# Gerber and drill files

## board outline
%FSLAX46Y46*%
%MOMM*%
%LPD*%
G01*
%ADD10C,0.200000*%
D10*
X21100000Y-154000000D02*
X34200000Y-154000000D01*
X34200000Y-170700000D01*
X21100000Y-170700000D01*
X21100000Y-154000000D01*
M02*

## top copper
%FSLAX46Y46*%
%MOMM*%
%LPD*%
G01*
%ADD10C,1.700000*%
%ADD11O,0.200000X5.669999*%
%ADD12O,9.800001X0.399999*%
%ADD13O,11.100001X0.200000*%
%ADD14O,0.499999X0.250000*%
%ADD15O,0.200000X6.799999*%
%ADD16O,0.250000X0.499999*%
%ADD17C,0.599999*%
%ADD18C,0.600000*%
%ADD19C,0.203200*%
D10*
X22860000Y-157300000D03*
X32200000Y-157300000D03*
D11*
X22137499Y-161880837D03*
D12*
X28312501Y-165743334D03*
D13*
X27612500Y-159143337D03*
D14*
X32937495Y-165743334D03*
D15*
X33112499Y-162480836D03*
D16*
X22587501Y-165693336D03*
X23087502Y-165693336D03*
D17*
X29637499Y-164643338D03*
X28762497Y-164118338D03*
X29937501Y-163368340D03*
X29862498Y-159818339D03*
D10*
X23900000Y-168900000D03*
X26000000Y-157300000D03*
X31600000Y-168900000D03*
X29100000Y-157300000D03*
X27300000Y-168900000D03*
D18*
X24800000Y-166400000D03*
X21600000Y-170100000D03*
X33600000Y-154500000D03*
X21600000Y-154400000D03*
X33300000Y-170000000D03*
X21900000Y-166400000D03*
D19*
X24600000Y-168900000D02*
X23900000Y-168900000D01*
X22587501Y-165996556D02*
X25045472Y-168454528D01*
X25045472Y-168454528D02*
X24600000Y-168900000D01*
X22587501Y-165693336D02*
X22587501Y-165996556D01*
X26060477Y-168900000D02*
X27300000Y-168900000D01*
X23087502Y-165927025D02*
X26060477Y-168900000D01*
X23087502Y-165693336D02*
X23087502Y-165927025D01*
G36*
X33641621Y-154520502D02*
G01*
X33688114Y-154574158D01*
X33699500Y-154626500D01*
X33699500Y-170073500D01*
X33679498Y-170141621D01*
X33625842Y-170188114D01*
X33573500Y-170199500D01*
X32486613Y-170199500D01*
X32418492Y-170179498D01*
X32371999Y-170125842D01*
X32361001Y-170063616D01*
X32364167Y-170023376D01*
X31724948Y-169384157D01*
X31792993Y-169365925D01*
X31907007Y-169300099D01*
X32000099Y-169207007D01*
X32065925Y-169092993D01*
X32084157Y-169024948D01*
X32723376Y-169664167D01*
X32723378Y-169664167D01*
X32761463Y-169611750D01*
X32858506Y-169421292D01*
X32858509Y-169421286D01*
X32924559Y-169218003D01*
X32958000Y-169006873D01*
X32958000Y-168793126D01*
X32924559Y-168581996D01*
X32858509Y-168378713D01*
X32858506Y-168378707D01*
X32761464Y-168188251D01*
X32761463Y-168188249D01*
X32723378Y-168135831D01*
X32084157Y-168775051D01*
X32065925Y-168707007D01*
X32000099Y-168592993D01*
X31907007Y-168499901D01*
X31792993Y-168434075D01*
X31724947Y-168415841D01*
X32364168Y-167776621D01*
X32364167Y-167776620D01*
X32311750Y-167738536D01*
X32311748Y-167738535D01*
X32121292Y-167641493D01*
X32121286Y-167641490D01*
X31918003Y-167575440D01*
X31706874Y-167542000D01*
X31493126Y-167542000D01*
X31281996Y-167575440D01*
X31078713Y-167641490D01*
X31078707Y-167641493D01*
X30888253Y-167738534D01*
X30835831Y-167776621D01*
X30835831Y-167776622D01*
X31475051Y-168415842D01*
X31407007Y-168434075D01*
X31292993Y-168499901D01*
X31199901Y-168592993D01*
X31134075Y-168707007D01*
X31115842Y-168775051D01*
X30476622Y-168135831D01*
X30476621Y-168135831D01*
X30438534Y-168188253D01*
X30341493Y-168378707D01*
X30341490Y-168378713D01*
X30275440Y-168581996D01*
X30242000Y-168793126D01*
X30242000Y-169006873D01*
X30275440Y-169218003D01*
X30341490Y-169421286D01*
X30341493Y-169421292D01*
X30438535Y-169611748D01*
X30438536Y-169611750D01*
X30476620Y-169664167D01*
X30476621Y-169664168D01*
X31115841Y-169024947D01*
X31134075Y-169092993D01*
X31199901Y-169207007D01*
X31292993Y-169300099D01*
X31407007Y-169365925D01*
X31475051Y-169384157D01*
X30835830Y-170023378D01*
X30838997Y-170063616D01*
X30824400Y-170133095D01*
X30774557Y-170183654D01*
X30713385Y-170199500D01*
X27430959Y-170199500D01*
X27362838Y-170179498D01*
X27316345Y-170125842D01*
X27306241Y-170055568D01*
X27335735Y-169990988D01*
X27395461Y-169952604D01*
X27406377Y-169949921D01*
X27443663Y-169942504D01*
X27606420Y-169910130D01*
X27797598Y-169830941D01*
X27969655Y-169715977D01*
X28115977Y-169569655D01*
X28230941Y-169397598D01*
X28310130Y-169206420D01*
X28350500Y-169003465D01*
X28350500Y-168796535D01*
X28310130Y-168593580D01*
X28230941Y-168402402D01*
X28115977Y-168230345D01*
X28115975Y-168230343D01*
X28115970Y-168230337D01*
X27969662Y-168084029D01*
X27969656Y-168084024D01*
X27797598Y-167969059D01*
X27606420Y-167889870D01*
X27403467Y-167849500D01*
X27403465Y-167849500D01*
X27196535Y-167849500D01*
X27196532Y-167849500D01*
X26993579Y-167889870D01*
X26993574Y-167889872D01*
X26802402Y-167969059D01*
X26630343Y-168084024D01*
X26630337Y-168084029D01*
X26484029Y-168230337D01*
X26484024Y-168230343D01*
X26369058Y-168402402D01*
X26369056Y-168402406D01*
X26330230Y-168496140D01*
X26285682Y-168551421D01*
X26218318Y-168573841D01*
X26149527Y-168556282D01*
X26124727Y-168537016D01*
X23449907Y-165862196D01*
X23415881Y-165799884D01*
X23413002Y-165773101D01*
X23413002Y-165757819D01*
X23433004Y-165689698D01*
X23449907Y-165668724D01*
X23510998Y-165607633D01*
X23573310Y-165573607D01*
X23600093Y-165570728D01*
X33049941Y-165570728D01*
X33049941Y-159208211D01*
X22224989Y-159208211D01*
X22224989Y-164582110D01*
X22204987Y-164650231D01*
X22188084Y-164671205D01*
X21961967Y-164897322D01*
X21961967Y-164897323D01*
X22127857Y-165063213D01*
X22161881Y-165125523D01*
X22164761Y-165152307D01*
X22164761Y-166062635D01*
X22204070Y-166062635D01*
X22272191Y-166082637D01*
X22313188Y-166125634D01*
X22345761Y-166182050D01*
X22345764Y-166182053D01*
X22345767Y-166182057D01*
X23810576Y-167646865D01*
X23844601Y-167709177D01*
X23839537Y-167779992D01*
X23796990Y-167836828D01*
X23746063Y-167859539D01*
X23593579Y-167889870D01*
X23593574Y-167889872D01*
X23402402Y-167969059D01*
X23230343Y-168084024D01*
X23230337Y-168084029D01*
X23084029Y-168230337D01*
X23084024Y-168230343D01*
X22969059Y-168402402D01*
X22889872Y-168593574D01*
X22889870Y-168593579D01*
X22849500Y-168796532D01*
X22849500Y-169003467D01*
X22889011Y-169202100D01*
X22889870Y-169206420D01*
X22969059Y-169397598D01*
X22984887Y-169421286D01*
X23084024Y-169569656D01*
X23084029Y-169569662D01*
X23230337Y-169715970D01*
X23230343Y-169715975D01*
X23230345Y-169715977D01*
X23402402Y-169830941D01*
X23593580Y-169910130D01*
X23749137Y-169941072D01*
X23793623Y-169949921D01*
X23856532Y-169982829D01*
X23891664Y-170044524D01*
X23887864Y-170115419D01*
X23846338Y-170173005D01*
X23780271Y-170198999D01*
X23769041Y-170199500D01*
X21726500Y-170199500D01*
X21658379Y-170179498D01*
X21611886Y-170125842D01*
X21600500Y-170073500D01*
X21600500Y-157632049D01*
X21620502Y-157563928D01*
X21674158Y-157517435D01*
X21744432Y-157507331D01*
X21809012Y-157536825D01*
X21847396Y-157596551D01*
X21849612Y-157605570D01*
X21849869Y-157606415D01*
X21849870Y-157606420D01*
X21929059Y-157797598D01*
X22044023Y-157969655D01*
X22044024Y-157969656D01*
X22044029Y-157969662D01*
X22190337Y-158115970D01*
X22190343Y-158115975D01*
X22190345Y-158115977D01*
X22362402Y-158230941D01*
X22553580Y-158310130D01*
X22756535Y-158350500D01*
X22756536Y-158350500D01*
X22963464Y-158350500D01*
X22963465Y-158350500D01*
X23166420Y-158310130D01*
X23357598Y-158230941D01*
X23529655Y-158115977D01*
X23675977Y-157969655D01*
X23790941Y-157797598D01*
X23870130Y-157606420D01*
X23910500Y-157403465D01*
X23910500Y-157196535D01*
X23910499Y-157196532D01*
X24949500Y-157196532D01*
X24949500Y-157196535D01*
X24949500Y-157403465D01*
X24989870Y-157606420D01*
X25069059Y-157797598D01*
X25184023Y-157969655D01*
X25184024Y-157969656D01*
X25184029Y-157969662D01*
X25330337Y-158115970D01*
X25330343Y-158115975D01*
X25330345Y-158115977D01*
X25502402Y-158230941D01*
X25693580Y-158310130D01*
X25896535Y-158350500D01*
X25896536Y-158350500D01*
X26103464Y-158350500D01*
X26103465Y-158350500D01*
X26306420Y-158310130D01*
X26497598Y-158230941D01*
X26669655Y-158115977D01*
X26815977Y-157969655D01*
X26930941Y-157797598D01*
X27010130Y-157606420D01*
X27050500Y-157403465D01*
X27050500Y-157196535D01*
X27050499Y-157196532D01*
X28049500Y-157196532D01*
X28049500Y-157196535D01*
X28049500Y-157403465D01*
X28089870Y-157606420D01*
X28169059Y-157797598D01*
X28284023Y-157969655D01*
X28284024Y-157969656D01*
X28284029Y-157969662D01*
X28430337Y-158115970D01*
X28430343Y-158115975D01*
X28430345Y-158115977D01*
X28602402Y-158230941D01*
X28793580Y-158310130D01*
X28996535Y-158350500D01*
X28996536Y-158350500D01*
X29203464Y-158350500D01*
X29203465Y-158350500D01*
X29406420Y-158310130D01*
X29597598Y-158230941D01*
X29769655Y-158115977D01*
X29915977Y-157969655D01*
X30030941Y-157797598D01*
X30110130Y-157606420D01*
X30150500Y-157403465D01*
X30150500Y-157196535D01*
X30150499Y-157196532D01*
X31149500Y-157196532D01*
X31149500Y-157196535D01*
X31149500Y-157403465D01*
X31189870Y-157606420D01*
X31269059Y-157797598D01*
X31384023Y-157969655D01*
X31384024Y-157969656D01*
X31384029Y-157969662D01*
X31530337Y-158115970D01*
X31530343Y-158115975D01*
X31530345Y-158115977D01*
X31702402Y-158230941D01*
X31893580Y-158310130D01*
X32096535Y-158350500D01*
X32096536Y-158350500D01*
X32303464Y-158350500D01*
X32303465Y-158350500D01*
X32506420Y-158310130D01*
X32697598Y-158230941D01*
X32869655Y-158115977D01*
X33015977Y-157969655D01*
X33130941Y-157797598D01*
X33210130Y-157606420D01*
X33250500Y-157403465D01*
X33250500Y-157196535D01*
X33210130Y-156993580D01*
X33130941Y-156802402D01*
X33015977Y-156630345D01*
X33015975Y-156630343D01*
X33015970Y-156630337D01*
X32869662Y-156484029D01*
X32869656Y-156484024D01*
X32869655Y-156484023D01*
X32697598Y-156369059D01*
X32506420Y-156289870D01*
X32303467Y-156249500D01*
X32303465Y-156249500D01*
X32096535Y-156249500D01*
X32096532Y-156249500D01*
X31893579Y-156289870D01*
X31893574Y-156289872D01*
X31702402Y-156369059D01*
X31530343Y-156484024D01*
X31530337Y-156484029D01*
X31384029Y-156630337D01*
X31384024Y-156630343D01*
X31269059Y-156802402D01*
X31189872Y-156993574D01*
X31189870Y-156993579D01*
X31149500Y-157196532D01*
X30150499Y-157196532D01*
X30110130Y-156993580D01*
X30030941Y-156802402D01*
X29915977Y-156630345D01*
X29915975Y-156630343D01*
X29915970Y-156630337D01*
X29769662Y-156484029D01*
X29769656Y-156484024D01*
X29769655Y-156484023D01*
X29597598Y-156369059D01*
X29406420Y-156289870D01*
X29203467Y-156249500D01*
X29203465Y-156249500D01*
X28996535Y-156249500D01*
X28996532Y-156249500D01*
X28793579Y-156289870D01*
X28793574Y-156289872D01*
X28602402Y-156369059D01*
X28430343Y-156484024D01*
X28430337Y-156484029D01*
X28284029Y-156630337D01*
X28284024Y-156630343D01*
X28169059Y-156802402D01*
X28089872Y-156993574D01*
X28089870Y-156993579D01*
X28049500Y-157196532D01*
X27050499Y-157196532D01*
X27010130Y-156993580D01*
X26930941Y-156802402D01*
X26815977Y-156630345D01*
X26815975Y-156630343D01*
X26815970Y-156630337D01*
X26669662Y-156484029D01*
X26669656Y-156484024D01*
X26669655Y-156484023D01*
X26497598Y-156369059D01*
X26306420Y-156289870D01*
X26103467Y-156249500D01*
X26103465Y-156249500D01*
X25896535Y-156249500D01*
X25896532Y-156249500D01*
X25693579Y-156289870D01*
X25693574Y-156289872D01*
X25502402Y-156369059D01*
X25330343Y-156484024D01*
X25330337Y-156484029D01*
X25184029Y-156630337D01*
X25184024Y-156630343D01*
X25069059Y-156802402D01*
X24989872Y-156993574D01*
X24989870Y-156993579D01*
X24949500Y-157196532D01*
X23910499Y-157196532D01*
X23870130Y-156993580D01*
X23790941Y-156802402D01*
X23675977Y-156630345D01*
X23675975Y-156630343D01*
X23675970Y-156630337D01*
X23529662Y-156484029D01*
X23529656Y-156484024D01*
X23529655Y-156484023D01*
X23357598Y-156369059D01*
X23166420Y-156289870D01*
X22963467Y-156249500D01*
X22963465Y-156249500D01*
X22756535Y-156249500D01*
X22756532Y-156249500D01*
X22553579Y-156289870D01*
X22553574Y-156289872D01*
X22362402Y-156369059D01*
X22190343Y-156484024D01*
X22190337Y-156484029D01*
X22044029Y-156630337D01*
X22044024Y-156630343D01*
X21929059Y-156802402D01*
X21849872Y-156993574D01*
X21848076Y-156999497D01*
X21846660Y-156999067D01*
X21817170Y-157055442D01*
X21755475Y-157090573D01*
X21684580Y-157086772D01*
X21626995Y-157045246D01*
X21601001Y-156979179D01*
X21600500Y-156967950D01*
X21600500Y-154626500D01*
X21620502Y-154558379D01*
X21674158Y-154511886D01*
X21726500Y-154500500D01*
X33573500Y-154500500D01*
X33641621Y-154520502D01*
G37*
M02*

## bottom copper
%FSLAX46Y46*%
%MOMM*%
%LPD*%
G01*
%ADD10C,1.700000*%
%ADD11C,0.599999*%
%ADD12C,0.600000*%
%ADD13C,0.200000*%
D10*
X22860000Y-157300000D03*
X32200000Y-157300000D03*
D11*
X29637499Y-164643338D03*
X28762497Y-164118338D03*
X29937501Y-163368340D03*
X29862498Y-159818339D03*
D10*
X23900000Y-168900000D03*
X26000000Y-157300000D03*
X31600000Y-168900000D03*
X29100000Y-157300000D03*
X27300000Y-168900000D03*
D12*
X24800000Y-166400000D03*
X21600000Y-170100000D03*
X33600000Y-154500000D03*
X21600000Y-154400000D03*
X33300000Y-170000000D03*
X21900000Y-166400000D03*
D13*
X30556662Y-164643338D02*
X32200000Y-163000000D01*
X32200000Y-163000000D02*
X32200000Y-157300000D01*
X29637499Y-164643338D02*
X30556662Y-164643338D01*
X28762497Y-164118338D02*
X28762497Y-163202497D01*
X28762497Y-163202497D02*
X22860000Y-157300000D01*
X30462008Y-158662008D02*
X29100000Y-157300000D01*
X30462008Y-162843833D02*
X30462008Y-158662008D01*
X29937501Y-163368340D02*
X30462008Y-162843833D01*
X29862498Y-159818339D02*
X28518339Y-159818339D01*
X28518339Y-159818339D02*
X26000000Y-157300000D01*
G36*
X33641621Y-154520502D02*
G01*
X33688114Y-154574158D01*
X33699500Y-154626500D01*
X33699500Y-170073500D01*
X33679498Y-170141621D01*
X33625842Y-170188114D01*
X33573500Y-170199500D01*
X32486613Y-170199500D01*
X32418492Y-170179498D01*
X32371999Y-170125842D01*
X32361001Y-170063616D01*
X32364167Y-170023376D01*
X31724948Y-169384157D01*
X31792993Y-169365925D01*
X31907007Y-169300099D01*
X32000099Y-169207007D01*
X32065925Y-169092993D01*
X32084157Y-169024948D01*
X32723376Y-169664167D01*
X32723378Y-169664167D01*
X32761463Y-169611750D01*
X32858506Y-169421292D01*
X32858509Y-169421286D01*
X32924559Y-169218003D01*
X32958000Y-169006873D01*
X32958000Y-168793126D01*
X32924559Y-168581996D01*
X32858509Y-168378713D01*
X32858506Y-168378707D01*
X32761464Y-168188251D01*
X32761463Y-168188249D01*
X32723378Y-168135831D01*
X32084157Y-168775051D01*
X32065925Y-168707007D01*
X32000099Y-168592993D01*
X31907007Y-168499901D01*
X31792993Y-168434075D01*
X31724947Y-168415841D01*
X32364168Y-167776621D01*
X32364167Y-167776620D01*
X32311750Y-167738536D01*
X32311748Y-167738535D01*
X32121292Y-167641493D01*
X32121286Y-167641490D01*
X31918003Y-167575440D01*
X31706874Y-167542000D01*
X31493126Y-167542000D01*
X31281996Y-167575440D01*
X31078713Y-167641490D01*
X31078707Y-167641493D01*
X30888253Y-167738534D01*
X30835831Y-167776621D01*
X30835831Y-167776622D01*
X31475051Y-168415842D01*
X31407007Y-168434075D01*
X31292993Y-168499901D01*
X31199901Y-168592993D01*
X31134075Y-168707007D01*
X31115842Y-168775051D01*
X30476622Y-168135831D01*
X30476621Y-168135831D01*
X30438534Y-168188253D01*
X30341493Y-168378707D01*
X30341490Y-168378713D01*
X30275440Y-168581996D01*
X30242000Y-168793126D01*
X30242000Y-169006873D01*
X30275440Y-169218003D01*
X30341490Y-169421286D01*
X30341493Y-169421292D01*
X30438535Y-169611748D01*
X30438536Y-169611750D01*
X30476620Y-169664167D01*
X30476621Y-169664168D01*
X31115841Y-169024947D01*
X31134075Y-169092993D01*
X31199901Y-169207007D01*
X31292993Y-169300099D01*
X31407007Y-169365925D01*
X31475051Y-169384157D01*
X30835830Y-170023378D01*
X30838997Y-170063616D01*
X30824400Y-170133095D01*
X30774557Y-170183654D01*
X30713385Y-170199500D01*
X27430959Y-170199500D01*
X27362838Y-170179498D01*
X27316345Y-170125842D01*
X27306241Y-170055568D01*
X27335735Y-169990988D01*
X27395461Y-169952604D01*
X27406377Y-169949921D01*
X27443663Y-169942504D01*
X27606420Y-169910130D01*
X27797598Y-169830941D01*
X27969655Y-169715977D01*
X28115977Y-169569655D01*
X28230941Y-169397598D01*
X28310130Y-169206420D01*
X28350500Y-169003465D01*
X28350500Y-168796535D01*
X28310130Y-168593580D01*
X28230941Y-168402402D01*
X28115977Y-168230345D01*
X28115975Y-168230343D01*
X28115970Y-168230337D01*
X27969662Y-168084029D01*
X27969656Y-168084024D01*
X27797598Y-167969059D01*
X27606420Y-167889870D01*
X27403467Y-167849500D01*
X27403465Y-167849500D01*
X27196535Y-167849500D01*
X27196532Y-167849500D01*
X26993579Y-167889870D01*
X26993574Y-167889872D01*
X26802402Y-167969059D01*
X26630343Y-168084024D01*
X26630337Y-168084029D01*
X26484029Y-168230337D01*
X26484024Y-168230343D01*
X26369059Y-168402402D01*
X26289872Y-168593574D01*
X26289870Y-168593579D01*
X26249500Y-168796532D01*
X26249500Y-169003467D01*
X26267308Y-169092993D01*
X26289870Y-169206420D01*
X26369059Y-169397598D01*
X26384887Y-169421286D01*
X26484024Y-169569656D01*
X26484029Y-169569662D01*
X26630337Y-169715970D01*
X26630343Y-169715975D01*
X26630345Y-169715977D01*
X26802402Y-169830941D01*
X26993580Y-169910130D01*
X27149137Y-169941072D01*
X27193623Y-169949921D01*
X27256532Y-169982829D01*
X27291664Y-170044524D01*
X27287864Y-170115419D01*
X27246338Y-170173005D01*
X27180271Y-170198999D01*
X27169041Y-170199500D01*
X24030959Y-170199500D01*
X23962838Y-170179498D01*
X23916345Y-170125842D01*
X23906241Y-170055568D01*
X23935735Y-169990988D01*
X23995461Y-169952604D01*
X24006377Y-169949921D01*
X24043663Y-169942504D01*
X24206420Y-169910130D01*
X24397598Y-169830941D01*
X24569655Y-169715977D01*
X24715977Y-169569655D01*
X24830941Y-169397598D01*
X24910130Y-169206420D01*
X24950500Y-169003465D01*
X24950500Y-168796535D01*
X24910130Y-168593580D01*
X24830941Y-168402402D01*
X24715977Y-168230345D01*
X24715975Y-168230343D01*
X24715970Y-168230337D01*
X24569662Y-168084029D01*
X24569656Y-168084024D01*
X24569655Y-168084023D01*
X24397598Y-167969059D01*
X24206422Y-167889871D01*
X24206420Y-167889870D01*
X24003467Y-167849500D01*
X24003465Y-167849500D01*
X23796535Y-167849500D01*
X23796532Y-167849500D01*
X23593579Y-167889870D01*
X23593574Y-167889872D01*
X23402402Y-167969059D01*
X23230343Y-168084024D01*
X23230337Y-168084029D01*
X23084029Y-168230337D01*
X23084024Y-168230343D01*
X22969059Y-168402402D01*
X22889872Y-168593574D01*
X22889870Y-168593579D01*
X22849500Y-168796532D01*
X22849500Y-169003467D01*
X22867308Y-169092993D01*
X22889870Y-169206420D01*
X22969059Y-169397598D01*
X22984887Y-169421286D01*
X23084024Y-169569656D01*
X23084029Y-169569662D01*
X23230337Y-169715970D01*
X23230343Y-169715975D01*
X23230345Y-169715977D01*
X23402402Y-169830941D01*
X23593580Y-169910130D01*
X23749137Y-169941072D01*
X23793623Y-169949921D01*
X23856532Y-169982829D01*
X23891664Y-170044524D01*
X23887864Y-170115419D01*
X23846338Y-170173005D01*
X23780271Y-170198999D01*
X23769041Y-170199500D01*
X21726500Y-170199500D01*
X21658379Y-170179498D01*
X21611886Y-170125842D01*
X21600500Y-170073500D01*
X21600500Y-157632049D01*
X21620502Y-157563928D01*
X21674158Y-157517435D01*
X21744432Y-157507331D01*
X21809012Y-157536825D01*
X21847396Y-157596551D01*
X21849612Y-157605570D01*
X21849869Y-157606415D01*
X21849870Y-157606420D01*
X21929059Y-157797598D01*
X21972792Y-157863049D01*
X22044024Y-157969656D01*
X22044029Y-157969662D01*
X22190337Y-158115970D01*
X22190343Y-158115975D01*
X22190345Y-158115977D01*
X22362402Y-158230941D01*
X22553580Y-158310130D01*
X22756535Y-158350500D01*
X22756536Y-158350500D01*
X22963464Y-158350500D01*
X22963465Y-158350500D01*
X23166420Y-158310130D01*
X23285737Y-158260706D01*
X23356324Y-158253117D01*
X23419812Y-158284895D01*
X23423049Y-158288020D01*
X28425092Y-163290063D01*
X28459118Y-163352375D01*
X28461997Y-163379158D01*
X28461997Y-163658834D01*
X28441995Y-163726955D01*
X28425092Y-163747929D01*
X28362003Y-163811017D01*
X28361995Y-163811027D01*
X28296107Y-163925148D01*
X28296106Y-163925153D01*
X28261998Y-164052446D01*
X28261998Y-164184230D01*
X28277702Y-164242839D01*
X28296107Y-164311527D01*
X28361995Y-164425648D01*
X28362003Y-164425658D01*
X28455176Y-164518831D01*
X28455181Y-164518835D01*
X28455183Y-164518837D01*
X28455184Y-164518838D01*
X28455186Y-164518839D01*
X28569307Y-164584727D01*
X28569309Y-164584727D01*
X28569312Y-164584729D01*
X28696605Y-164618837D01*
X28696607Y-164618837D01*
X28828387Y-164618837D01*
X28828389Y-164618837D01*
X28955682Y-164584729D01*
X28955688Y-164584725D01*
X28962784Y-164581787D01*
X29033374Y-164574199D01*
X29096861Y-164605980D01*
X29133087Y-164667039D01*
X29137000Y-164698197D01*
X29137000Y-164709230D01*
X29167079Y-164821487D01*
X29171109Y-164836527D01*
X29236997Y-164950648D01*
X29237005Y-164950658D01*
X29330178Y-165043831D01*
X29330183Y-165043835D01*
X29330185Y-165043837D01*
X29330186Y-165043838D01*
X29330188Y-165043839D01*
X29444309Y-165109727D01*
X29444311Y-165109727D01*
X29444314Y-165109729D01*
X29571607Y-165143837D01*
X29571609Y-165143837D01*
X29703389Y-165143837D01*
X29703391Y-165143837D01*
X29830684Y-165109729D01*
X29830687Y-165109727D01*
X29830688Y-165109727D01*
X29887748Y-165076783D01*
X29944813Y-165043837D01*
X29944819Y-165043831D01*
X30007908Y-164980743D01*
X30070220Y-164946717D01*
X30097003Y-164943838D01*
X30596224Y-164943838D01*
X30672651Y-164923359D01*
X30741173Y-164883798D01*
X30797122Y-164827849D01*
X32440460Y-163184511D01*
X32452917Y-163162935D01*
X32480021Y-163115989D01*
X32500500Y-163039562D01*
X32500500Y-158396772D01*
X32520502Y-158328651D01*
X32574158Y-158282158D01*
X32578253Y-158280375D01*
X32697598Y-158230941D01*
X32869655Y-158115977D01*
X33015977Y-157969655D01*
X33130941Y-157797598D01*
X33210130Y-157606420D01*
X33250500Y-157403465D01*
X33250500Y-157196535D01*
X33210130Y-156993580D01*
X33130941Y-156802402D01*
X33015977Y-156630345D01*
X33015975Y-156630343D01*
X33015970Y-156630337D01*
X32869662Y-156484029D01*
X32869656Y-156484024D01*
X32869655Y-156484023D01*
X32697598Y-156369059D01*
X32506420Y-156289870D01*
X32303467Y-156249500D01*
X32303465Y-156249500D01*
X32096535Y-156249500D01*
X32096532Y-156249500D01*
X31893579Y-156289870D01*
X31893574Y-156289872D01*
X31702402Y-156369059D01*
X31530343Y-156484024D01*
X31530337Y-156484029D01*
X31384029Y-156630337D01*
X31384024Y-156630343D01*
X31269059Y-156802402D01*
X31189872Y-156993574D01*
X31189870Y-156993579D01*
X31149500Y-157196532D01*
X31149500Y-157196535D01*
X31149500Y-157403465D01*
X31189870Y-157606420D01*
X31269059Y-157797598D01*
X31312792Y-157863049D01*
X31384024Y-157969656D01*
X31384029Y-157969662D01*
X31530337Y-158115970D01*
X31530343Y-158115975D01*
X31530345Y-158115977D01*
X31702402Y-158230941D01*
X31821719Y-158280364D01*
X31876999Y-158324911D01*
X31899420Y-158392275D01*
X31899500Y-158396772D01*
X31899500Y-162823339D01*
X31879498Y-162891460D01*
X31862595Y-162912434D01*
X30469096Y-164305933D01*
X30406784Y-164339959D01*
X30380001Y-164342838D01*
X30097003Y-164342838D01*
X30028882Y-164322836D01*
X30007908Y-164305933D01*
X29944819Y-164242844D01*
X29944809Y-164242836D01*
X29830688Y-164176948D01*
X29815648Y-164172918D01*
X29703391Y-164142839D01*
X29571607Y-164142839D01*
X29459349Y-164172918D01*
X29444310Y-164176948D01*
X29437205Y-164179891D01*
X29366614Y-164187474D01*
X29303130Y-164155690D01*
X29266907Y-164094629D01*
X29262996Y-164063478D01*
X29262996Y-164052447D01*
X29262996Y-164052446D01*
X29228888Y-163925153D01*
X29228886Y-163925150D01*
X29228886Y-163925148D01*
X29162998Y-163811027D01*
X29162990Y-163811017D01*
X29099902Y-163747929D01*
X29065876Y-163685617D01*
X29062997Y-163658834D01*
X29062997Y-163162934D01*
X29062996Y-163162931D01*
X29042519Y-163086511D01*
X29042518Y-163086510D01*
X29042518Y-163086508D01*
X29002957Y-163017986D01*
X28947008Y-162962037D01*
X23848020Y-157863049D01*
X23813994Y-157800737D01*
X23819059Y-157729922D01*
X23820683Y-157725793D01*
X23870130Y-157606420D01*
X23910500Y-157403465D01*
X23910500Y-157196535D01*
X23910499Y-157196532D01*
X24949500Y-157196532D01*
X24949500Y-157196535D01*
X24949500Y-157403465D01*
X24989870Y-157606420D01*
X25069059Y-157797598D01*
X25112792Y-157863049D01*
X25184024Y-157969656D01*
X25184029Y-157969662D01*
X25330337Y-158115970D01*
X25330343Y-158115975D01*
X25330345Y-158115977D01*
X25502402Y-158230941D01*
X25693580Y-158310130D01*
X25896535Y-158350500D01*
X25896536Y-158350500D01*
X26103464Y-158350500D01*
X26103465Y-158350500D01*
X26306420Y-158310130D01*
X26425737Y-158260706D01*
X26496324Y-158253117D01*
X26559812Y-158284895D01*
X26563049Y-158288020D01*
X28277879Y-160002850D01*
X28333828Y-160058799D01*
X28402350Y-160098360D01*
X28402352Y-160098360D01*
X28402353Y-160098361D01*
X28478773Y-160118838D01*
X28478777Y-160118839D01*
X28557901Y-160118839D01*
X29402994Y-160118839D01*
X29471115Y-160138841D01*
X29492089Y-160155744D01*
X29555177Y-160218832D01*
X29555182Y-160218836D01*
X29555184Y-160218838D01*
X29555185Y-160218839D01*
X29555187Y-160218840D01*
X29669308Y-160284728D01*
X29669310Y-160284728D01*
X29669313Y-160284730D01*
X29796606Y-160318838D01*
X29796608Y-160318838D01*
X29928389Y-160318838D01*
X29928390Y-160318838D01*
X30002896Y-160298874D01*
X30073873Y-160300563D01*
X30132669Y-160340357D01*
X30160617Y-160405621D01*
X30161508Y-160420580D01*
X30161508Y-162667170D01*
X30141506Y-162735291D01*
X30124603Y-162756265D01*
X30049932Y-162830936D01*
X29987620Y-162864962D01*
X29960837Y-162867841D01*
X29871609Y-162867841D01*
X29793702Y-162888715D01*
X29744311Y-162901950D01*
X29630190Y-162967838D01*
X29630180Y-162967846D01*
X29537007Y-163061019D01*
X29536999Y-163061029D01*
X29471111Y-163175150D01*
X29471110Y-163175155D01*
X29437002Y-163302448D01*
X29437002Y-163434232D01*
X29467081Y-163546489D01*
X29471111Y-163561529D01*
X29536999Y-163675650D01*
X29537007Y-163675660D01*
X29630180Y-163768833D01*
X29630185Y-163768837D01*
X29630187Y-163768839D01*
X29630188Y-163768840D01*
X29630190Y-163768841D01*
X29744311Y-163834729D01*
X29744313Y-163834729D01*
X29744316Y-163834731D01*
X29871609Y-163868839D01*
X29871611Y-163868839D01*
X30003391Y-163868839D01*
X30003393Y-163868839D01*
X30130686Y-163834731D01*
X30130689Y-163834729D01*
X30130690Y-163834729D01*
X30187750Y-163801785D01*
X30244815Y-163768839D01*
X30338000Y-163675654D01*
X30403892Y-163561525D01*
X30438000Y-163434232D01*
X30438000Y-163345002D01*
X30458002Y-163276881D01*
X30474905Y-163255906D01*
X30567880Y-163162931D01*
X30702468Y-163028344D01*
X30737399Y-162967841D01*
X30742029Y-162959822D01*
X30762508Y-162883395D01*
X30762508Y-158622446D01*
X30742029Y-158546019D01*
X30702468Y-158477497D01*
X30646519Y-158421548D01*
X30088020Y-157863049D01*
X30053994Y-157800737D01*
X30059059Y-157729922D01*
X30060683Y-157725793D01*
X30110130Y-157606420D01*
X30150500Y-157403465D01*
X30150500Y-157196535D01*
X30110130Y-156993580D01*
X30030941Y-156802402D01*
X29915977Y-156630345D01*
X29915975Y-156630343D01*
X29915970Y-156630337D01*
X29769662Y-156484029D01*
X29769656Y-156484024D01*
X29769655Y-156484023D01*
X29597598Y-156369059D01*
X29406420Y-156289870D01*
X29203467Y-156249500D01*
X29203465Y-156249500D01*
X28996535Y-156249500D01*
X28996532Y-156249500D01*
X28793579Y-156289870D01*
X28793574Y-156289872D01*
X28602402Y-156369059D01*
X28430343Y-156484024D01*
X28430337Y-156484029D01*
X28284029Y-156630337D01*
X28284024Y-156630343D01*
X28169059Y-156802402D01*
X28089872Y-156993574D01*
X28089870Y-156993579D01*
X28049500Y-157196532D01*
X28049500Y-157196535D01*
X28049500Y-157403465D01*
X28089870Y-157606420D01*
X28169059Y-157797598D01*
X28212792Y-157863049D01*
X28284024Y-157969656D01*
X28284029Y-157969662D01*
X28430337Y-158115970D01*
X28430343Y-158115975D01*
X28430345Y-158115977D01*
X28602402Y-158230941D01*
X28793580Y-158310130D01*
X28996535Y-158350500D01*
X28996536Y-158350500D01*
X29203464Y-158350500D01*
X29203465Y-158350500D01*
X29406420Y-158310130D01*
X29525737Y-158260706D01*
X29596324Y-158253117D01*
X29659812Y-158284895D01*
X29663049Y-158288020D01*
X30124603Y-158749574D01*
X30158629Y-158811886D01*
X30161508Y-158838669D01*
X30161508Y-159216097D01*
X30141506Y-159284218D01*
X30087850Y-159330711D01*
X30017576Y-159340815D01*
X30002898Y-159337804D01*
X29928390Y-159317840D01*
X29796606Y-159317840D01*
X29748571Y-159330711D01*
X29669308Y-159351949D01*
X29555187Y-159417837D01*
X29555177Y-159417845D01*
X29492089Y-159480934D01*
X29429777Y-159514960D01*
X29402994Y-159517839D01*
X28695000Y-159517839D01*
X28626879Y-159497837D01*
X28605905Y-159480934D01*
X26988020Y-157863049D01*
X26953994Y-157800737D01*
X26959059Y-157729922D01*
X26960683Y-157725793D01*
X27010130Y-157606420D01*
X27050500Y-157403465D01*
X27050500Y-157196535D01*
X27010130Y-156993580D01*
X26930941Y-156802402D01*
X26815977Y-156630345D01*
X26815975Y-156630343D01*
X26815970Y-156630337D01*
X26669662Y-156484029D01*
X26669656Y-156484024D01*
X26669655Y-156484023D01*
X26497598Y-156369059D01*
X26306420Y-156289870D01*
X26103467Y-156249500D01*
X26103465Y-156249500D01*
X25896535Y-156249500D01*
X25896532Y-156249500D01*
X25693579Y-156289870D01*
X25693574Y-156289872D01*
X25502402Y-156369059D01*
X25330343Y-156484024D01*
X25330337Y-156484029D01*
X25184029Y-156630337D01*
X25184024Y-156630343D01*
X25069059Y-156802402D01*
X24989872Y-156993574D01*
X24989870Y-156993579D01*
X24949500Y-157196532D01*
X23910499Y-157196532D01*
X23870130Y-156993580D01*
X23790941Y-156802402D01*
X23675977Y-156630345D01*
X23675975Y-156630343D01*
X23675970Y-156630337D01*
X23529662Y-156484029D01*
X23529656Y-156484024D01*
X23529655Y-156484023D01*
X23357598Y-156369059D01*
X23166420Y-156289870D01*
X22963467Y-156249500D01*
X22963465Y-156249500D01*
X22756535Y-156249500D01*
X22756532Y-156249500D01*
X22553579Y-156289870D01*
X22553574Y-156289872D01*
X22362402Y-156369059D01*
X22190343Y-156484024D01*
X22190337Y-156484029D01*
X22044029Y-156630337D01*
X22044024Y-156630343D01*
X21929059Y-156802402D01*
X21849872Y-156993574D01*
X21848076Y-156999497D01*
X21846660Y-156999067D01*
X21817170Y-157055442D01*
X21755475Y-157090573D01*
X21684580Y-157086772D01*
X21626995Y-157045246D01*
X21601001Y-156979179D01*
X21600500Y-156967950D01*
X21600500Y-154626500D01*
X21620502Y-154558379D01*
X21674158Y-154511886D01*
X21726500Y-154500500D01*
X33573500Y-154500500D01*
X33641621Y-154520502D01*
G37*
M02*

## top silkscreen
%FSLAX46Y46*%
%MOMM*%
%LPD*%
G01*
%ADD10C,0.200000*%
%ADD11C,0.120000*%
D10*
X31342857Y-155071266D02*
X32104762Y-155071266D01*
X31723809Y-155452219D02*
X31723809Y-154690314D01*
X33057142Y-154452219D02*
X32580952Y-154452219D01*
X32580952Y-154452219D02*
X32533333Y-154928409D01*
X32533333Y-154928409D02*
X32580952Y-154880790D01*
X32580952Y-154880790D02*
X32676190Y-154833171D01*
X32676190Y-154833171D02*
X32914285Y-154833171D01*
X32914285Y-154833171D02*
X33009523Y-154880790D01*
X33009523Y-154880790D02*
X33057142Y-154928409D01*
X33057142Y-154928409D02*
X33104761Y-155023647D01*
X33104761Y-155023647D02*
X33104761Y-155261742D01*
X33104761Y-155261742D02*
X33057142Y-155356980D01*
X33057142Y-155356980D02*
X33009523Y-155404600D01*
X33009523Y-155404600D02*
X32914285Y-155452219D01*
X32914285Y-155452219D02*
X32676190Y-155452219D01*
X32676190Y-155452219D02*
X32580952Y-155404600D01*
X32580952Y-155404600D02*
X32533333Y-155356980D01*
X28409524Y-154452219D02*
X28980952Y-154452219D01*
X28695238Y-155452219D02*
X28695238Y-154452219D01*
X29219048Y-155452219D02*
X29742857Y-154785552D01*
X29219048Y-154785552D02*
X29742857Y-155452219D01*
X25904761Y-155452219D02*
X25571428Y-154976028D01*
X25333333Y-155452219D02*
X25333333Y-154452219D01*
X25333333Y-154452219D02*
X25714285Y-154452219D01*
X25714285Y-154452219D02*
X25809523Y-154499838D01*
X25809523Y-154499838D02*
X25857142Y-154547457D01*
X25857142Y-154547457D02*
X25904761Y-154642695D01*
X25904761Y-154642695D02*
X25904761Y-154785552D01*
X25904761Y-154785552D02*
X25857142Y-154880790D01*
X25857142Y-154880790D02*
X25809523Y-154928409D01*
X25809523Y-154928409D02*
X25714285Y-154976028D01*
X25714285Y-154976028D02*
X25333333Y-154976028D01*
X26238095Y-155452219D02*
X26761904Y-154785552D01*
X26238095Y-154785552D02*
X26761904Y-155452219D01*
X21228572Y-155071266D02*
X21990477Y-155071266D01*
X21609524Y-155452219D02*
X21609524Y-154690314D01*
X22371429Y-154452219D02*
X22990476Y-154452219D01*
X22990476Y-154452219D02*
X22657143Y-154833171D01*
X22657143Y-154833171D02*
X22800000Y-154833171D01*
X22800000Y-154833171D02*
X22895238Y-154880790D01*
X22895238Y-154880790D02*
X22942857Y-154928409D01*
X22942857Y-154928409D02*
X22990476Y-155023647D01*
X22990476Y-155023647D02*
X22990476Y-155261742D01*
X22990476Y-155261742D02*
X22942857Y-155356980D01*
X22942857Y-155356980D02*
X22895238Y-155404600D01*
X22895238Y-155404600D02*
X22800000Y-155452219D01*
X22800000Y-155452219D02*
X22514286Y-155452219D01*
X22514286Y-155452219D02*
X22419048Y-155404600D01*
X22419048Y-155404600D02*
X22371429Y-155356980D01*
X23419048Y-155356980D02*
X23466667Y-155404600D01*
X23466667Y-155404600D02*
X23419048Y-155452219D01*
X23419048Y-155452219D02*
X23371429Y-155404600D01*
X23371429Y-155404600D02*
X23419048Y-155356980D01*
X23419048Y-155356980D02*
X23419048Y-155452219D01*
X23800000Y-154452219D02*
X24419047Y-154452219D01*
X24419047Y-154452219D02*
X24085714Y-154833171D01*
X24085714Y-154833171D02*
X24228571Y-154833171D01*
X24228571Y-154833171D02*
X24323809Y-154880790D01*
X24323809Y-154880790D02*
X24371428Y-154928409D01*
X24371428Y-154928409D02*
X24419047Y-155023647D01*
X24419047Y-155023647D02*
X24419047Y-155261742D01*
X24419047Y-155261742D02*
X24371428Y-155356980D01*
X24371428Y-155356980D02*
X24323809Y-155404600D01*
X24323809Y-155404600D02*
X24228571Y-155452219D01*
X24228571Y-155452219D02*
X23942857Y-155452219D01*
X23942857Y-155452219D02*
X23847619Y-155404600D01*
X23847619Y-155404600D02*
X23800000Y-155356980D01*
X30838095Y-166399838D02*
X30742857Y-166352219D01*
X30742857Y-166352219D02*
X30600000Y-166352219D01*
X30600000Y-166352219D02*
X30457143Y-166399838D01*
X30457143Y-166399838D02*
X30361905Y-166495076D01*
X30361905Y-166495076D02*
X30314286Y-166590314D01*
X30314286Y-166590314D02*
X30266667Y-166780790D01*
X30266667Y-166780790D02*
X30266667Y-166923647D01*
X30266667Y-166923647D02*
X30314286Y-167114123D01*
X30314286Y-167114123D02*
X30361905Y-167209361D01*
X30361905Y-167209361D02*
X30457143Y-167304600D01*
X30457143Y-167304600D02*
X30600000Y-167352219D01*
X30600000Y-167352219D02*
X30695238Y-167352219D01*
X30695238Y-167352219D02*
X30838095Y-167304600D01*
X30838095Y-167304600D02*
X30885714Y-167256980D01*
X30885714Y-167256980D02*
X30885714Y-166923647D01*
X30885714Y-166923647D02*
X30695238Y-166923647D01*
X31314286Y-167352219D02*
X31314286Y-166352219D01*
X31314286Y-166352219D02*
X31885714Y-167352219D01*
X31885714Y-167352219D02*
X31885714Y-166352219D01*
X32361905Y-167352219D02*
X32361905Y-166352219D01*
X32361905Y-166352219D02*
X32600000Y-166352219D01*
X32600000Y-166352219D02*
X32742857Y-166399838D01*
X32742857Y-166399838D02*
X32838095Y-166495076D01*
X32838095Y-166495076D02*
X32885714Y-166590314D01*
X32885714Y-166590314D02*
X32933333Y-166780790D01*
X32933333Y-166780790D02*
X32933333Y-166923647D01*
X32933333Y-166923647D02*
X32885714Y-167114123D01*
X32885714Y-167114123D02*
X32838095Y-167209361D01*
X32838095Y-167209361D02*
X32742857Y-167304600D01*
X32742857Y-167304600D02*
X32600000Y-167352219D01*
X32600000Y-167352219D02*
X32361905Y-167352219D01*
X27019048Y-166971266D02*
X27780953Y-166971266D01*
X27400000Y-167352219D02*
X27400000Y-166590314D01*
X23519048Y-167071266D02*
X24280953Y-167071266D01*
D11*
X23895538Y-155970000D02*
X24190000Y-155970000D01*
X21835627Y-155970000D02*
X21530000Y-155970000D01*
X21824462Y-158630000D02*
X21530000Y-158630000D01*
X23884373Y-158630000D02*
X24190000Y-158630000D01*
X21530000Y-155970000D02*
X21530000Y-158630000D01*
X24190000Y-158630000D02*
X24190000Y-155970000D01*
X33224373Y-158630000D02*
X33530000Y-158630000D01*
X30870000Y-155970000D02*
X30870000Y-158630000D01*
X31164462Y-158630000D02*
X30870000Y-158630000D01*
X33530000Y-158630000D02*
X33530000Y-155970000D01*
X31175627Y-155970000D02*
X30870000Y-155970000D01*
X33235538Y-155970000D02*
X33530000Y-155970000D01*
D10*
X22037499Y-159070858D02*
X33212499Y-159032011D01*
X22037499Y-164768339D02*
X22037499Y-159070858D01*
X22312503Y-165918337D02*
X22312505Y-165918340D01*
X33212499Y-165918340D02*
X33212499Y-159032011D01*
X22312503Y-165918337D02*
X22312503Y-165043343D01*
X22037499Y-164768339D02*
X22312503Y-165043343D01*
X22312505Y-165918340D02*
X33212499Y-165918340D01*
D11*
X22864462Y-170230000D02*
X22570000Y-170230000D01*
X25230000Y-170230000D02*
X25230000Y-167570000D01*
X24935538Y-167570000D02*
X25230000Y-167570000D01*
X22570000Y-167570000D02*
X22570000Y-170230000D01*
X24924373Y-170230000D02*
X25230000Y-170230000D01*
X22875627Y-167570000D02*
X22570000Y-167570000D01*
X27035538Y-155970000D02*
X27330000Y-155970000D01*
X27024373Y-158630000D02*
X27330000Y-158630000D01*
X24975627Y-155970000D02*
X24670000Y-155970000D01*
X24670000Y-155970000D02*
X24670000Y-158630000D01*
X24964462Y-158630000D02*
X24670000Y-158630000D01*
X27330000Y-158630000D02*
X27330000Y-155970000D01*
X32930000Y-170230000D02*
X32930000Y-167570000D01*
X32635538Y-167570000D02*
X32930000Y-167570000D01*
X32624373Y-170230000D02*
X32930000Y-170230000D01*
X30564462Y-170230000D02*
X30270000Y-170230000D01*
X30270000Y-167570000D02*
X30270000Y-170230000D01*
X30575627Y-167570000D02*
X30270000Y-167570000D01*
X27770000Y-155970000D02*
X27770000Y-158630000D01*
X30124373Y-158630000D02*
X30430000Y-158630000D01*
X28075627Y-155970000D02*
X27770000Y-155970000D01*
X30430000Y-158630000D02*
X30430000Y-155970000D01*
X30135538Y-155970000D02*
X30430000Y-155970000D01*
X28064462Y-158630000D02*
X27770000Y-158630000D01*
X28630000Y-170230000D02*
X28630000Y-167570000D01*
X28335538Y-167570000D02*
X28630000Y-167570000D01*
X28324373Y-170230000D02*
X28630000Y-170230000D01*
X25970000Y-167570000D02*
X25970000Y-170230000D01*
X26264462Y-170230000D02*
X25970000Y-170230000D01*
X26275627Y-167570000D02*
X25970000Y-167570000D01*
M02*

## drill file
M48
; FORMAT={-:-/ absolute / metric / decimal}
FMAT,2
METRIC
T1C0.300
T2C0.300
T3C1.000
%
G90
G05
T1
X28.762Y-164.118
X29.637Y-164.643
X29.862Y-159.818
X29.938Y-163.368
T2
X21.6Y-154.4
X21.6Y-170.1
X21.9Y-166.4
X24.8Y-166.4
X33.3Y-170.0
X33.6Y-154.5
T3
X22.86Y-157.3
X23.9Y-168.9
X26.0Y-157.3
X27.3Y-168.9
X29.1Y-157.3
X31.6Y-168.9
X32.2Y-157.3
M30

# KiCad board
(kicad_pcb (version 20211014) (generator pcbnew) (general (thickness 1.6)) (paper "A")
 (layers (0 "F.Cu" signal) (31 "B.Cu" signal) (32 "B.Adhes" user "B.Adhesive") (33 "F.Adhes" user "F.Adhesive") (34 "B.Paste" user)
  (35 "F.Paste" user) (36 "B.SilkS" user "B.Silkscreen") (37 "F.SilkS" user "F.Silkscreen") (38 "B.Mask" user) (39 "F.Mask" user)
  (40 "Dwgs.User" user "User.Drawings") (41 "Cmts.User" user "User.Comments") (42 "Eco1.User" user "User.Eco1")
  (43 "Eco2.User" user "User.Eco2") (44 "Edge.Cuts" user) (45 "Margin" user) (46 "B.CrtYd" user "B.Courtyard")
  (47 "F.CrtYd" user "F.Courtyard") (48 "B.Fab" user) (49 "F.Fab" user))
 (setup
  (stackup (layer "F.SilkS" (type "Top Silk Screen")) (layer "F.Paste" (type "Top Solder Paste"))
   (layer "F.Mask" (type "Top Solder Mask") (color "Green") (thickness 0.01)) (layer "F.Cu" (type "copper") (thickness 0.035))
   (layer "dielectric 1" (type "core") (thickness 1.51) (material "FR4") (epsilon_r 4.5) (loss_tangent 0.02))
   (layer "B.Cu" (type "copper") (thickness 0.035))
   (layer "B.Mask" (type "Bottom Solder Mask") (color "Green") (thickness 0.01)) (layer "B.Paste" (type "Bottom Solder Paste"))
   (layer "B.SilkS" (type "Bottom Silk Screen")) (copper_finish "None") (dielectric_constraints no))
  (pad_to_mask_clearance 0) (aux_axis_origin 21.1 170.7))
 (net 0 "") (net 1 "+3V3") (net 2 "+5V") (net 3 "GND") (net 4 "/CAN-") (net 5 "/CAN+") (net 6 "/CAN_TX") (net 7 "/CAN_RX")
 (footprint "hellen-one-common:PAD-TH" (layer "F.Cu") (at 22.86 157.3)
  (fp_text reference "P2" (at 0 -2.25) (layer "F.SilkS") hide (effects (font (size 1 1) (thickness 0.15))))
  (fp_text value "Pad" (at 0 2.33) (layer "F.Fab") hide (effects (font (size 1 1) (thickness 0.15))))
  (fp_line (start 1.035538 -1.33) (end 1.33 -1.33) (layer "F.SilkS") (width 0.12))
  (fp_line (start -1.024373 -1.33) (end -1.33 -1.33) (layer "F.SilkS") (width 0.12))
  (fp_line (start -1.035538 1.33) (end -1.33 1.33) (layer "F.SilkS") (width 0.12))
  (fp_line (start 1.024373 1.33) (end 1.33 1.33) (layer "F.SilkS") (width 0.12))
  (fp_line (start -1.33 -1.33) (end -1.33 1.33) (layer "F.SilkS") (width 0.12))
  (fp_line (start 1.33 1.33) (end 1.33 -1.33) (layer "F.SilkS") (width 0.12))
  (pad "1" thru_hole circle locked (at 0 0) (size 1.7 1.7) (drill 1) (layers *.Cu *.Mask) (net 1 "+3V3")))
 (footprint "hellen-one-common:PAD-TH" (layer "F.Cu") (at 32.2 157.3)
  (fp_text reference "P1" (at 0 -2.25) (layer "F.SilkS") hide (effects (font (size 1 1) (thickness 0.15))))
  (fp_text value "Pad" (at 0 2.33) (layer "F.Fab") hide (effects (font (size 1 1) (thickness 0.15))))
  (fp_line (start 1.024373 1.33) (end 1.33 1.33) (layer "F.SilkS") (width 0.12))
  (fp_line (start -1.33 -1.33) (end -1.33 1.33) (layer "F.SilkS") (width 0.12))
  (fp_line (start -1.035538 1.33) (end -1.33 1.33) (layer "F.SilkS") (width 0.12))
  (fp_line (start 1.33 1.33) (end 1.33 -1.33) (layer "F.SilkS") (width 0.12))
  (fp_line (start -1.024373 -1.33) (end -1.33 -1.33) (layer "F.SilkS") (width 0.12))
  (fp_line (start 1.035538 -1.33) (end 1.33 -1.33) (layer "F.SilkS") (width 0.12))
  (pad "1" thru_hole circle locked (at 0 0) (size 1.7 1.7) (drill 1) (layers *.Cu *.Mask) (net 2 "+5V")))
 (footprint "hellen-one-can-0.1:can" (layer "F.Cu") (at 21.937502 166.018337) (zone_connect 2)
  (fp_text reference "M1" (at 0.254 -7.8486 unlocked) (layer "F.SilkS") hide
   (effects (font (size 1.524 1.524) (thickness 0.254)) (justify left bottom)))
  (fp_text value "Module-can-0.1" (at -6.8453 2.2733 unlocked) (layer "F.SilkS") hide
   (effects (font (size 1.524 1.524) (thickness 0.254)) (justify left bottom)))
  (fp_line (start 0.099997 -6.947479) (end 11.274997 -6.986326) (layer "F.SilkS") (width 0.2))
  (fp_line (start 0.099997 -1.249998) (end 0.099997 -6.947479) (layer "F.SilkS") (width 0.2))
  (fp_line (start 0.375001 -0.1) (end 0.375003 -0.099997) (layer "F.SilkS") (width 0.2))
  (fp_line (start 11.274997 -0.099997) (end 11.274997 -6.986326) (layer "F.SilkS") (width 0.2))
  (fp_line (start 0.375001 -0.1) (end 0.375001 -0.974994) (layer "F.SilkS") (width 0.2))
  (fp_line (start 0.099997 -1.249998) (end 0.375001 -0.974994) (layer "F.SilkS") (width 0.2))
  (fp_line (start 0.375003 -0.099997) (end 11.274997 -0.099997) (layer "F.SilkS") (width 0.2))
  (pad "E1" smd oval locked (at 0.199997 -4.1375 180) (size 0.2 5.669999) (layers "F.Cu" "F.Paste") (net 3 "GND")
   (solder_mask_margin 0.1016) (solder_paste_margin -49.999999) (zone_connect 2))
  (pad "E1" smd oval locked (at 6.374999 -0.275003 270) (size 0.399999 9.800001) (layers "F.Cu" "F.Paste") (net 3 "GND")
   (solder_mask_margin 0.1016) (solder_paste_margin -49.999999) (zone_connect 2))
  (pad "E1" smd oval locked (at 5.674998 -6.875 90) (size 0.2 11.100001) (layers "F.Cu" "F.Paste") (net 3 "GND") (solder_mask_margin 0.1016)
   (solder_paste_margin -49.999999) (zone_connect 2))
  (pad "E1" smd oval locked (at 10.999993 -0.275003 180) (size 0.499999 0.25) (layers "F.Cu" "F.Paste" "F.Mask") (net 3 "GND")
   (solder_paste_margin -49.999999) (zone_connect 2))
  (pad "E1" smd oval locked (at 11.174997 -3.537501 180) (size 0.2 6.799999) (layers "F.Cu" "F.Paste") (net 3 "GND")
   (solder_mask_margin 0.1016) (solder_paste_margin -49.999999) (zone_connect 2))
  (pad "S1" smd oval locked (at 0.649999 -0.325001) (size 0.25 0.499999) (layers "F.Cu" "F.Paste" "F.Mask") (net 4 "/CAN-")
   (solder_paste_margin -49.999999) (zone_connect 2))
  (pad "S2" smd oval locked (at 1.15 -0.325001) (size 0.25 0.499999) (layers "F.Cu" "F.Paste" "F.Mask") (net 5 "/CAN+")
   (solder_paste_margin -49.999999) (zone_connect 2))
  (pad "V1" thru_hole circle locked (at 7.699997 -1.374999 180) (size 0.599999 0.599999) (drill 0.299999) (layers *.Cu *.Mask) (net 2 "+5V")
   (solder_paste_margin -49.999999) (zone_connect 2))
  (pad "V2" thru_hole circle locked (at 6.824995 -1.899999 180) (size 0.599999 0.599999) (drill 0.299999) (layers *.Cu *.Mask)
   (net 1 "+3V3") (solder_paste_margin -49.999999) (zone_connect 2))
  (pad "V5" thru_hole circle locked (at 7.999999 -2.649997 270) (size 0.599999 0.599999) (drill 0.299999) (layers *.Cu *.Mask)
   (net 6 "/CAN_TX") (solder_paste_margin -49.999999) (zone_connect 2))
  (pad "V6" thru_hole circle locked (at 7.924996 -6.199998 270) (size 0.599999 0.599999) (drill 0.299999) (layers *.Cu *.Mask)
   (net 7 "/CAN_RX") (solder_paste_margin -49.999999) (zone_connect 2))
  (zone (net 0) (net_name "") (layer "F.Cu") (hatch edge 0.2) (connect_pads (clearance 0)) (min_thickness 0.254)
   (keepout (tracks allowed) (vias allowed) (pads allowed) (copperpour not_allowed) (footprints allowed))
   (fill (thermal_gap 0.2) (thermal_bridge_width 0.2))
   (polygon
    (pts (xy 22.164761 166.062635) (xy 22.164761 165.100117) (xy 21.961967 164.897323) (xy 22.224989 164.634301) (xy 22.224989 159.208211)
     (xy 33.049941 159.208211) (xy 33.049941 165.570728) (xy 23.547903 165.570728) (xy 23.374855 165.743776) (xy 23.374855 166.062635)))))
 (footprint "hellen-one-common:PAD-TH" (layer "F.Cu") (at 23.9 168.9)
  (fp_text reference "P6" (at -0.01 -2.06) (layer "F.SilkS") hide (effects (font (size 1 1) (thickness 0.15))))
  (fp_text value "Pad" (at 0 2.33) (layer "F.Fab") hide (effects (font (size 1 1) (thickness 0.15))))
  (fp_line (start -1.035538 1.33) (end -1.33 1.33) (layer "F.SilkS") (width 0.12))
  (fp_line (start 1.33 1.33) (end 1.33 -1.33) (layer "F.SilkS") (width 0.12))
  (fp_line (start 1.035538 -1.33) (end 1.33 -1.33) (layer "F.SilkS") (width 0.12))
  (fp_line (start -1.33 -1.33) (end -1.33 1.33) (layer "F.SilkS") (width 0.12))
  (fp_line (start 1.024373 1.33) (end 1.33 1.33) (layer "F.SilkS") (width 0.12))
  (fp_line (start -1.024373 -1.33) (end -1.33 -1.33) (layer "F.SilkS") (width 0.12))
  (pad "1" thru_hole circle locked (at 0 0) (size 1.7 1.7) (drill 1) (layers *.Cu *.Mask) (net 4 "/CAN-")))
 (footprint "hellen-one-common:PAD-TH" (layer "F.Cu") (at 26 157.3)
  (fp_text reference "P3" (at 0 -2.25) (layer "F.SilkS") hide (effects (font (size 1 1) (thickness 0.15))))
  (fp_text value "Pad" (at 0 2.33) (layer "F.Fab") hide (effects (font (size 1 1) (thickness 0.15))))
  (fp_line (start 1.035538 -1.33) (end 1.33 -1.33) (layer "F.SilkS") (width 0.12))
  (fp_line (start 1.024373 1.33) (end 1.33 1.33) (layer "F.SilkS") (width 0.12))
  (fp_line (start -1.024373 -1.33) (end -1.33 -1.33) (layer "F.SilkS") (width 0.12))
  (fp_line (start -1.33 -1.33) (end -1.33 1.33) (layer "F.SilkS") (width 0.12))
  (fp_line (start -1.035538 1.33) (end -1.33 1.33) (layer "F.SilkS") (width 0.12))
  (fp_line (start 1.33 1.33) (end 1.33 -1.33) (layer "F.SilkS") (width 0.12))
  (pad "1" thru_hole circle locked (at 0 0) (size 1.7 1.7) (drill 1) (layers *.Cu *.Mask) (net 7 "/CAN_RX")))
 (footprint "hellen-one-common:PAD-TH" (layer "F.Cu") (at 31.6 168.9)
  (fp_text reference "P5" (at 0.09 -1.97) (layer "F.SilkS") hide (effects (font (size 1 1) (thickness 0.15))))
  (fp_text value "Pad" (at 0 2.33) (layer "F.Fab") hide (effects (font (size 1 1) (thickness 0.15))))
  (fp_line (start 1.33 1.33) (end 1.33 -1.33) (layer "F.SilkS") (width 0.12))
  (fp_line (start 1.035538 -1.33) (end 1.33 -1.33) (layer "F.SilkS") (width 0.12))
  (fp_line (start 1.024373 1.33) (end 1.33 1.33) (layer "F.SilkS") (width 0.12))
  (fp_line (start -1.035538 1.33) (end -1.33 1.33) (layer "F.SilkS") (width 0.12))
  (fp_line (start -1.33 -1.33) (end -1.33 1.33) (layer "F.SilkS") (width 0.12))
  (fp_line (start -1.024373 -1.33) (end -1.33 -1.33) (layer "F.SilkS") (width 0.12))
  (pad "1" thru_hole circle locked (at 0 0) (size 1.7 1.7) (drill 1) (layers *.Cu *.Mask) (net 3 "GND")))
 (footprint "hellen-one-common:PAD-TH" (layer "F.Cu") (at 29.1 157.3)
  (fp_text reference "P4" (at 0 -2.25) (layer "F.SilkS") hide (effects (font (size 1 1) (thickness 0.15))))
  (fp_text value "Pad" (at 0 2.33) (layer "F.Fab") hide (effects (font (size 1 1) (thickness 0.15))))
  (fp_line (start -1.33 -1.33) (end -1.33 1.33) (layer "F.SilkS") (width 0.12))
  (fp_line (start 1.024373 1.33) (end 1.33 1.33) (layer "F.SilkS") (width 0.12))
  (fp_line (start -1.024373 -1.33) (end -1.33 -1.33) (layer "F.SilkS") (width 0.12))
  (fp_line (start 1.33 1.33) (end 1.33 -1.33) (layer "F.SilkS") (width 0.12))
  (fp_line (start 1.035538 -1.33) (end 1.33 -1.33) (layer "F.SilkS") (width 0.12))
  (fp_line (start -1.035538 1.33) (end -1.33 1.33) (layer "F.SilkS") (width 0.12))
  (pad "1" thru_hole circle locked (at 0 0) (size 1.7 1.7) (drill 1) (layers *.Cu *.Mask) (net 6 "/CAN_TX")))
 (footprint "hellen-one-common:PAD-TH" (layer "F.Cu") (at 27.3 168.9)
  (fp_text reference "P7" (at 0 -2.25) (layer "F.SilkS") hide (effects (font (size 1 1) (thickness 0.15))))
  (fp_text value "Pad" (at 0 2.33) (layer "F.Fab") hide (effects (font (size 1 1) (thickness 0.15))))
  (fp_line (start 1.33 1.33) (end 1.33 -1.33) (layer "F.SilkS") (width 0.12))
  (fp_line (start 1.035538 -1.33) (end 1.33 -1.33) (layer "F.SilkS") (width 0.12))
  (fp_line (start 1.024373 1.33) (end 1.33 1.33) (layer "F.SilkS") (width 0.12))
  (fp_line (start -1.33 -1.33) (end -1.33 1.33) (layer "F.SilkS") (width 0.12))
  (fp_line (start -1.035538 1.33) (end -1.33 1.33) (layer "F.SilkS") (width 0.12))
  (fp_line (start -1.024373 -1.33) (end -1.33 -1.33) (layer "F.SilkS") (width 0.12))
  (pad "1" thru_hole circle locked (at 0 0) (size 1.7 1.7) (drill 1) (layers *.Cu *.Mask) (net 5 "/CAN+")))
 (gr_rect (start 21.1 170.7) (end 34.2 154) (layer "Edge.Cuts") (width 0.2) (fill none))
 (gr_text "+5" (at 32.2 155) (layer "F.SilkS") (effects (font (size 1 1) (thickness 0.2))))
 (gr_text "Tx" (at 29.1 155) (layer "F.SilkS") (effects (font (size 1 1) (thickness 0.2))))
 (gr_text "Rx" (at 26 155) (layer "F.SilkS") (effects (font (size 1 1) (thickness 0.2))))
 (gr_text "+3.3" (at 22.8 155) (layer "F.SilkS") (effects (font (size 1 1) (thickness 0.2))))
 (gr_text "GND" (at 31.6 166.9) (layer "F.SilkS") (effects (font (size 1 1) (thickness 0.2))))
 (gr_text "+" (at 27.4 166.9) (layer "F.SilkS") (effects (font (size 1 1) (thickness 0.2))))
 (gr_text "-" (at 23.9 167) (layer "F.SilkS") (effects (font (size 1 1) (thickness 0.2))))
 (via (at 24.8 166.4) (size 0.6) (drill 0.3) (layers "F.Cu" "B.Cu") (free) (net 3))
 (via (at 21.6 170.1) (size 0.6) (drill 0.3) (layers "F.Cu" "B.Cu") (free) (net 3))
 (via (at 33.6 154.5) (size 0.6) (drill 0.3) (layers "F.Cu" "B.Cu") (free) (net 3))
 (via (at 21.6 154.4) (size 0.6) (drill 0.3) (layers "F.Cu" "B.Cu") (free) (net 3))
 (via (at 33.3 170) (size 0.6) (drill 0.3) (layers "F.Cu" "B.Cu") (free) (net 3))
 (via (at 21.9 166.4) (size 0.6) (drill 0.3) (layers "F.Cu" "B.Cu") (free) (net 3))
 (segment (start 24.6 168.9) (end 23.9 168.9) (width 0.2032) (layer "F.Cu") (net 4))
 (segment (start 22.587501 165.996556) (end 25.045472 168.454528) (width 0.2032) (layer "F.Cu") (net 4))
 (segment (start 25.045472 168.454528) (end 24.6 168.9) (width 0.2032) (layer "F.Cu") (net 4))
 (segment (start 22.587501 165.693336) (end 22.587501 165.996556) (width 0.2032) (layer "F.Cu") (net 4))
 (segment (start 26.060477 168.9) (end 27.3 168.9) (width 0.2032) (layer "F.Cu") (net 5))
 (segment (start 23.087502 165.927025) (end 26.060477 168.9) (width 0.2032) (layer "F.Cu") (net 5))
 (segment (start 23.087502 165.693336) (end 23.087502 165.927025) (width 0.2032) (layer "F.Cu") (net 5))
 (segment (start 30.556662 164.643338) (end 32.2 163) (width 0.2) (layer "B.Cu") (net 2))
 (segment (start 32.2 163) (end 32.2 157.3) (width 0.2) (layer "B.Cu") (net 2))
 (segment (start 29.637499 164.643338) (end 30.556662 164.643338) (width 0.2) (layer "B.Cu") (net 2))
 (segment (start 28.762497 164.118338) (end 28.762497 163.202497) (width 0.2) (layer "B.Cu") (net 1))
 (segment (start 28.762497 163.202497) (end 22.86 157.3) (width 0.2) (layer "B.Cu") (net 1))
 (segment (start 30.462008 158.662008) (end 29.1 157.3) (width 0.2) (layer "B.Cu") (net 6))
 (segment (start 30.462008 162.843833) (end 30.462008 158.662008) (width 0.2) (layer "B.Cu") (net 6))
 (segment (start 29.937501 163.36834) (end 30.462008 162.843833) (width 0.2) (layer "B.Cu") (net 6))
 (segment (start 29.862498 159.818339) (end 28.518339 159.818339) (width 0.2) (layer "B.Cu") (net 7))
 (segment (start 28.518339 159.818339) (end 26 157.3) (width 0.2) (layer "B.Cu") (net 7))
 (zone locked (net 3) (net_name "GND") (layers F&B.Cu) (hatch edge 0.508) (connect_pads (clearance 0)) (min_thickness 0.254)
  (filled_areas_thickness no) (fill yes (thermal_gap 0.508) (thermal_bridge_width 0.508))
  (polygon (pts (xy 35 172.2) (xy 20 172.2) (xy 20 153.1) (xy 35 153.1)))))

